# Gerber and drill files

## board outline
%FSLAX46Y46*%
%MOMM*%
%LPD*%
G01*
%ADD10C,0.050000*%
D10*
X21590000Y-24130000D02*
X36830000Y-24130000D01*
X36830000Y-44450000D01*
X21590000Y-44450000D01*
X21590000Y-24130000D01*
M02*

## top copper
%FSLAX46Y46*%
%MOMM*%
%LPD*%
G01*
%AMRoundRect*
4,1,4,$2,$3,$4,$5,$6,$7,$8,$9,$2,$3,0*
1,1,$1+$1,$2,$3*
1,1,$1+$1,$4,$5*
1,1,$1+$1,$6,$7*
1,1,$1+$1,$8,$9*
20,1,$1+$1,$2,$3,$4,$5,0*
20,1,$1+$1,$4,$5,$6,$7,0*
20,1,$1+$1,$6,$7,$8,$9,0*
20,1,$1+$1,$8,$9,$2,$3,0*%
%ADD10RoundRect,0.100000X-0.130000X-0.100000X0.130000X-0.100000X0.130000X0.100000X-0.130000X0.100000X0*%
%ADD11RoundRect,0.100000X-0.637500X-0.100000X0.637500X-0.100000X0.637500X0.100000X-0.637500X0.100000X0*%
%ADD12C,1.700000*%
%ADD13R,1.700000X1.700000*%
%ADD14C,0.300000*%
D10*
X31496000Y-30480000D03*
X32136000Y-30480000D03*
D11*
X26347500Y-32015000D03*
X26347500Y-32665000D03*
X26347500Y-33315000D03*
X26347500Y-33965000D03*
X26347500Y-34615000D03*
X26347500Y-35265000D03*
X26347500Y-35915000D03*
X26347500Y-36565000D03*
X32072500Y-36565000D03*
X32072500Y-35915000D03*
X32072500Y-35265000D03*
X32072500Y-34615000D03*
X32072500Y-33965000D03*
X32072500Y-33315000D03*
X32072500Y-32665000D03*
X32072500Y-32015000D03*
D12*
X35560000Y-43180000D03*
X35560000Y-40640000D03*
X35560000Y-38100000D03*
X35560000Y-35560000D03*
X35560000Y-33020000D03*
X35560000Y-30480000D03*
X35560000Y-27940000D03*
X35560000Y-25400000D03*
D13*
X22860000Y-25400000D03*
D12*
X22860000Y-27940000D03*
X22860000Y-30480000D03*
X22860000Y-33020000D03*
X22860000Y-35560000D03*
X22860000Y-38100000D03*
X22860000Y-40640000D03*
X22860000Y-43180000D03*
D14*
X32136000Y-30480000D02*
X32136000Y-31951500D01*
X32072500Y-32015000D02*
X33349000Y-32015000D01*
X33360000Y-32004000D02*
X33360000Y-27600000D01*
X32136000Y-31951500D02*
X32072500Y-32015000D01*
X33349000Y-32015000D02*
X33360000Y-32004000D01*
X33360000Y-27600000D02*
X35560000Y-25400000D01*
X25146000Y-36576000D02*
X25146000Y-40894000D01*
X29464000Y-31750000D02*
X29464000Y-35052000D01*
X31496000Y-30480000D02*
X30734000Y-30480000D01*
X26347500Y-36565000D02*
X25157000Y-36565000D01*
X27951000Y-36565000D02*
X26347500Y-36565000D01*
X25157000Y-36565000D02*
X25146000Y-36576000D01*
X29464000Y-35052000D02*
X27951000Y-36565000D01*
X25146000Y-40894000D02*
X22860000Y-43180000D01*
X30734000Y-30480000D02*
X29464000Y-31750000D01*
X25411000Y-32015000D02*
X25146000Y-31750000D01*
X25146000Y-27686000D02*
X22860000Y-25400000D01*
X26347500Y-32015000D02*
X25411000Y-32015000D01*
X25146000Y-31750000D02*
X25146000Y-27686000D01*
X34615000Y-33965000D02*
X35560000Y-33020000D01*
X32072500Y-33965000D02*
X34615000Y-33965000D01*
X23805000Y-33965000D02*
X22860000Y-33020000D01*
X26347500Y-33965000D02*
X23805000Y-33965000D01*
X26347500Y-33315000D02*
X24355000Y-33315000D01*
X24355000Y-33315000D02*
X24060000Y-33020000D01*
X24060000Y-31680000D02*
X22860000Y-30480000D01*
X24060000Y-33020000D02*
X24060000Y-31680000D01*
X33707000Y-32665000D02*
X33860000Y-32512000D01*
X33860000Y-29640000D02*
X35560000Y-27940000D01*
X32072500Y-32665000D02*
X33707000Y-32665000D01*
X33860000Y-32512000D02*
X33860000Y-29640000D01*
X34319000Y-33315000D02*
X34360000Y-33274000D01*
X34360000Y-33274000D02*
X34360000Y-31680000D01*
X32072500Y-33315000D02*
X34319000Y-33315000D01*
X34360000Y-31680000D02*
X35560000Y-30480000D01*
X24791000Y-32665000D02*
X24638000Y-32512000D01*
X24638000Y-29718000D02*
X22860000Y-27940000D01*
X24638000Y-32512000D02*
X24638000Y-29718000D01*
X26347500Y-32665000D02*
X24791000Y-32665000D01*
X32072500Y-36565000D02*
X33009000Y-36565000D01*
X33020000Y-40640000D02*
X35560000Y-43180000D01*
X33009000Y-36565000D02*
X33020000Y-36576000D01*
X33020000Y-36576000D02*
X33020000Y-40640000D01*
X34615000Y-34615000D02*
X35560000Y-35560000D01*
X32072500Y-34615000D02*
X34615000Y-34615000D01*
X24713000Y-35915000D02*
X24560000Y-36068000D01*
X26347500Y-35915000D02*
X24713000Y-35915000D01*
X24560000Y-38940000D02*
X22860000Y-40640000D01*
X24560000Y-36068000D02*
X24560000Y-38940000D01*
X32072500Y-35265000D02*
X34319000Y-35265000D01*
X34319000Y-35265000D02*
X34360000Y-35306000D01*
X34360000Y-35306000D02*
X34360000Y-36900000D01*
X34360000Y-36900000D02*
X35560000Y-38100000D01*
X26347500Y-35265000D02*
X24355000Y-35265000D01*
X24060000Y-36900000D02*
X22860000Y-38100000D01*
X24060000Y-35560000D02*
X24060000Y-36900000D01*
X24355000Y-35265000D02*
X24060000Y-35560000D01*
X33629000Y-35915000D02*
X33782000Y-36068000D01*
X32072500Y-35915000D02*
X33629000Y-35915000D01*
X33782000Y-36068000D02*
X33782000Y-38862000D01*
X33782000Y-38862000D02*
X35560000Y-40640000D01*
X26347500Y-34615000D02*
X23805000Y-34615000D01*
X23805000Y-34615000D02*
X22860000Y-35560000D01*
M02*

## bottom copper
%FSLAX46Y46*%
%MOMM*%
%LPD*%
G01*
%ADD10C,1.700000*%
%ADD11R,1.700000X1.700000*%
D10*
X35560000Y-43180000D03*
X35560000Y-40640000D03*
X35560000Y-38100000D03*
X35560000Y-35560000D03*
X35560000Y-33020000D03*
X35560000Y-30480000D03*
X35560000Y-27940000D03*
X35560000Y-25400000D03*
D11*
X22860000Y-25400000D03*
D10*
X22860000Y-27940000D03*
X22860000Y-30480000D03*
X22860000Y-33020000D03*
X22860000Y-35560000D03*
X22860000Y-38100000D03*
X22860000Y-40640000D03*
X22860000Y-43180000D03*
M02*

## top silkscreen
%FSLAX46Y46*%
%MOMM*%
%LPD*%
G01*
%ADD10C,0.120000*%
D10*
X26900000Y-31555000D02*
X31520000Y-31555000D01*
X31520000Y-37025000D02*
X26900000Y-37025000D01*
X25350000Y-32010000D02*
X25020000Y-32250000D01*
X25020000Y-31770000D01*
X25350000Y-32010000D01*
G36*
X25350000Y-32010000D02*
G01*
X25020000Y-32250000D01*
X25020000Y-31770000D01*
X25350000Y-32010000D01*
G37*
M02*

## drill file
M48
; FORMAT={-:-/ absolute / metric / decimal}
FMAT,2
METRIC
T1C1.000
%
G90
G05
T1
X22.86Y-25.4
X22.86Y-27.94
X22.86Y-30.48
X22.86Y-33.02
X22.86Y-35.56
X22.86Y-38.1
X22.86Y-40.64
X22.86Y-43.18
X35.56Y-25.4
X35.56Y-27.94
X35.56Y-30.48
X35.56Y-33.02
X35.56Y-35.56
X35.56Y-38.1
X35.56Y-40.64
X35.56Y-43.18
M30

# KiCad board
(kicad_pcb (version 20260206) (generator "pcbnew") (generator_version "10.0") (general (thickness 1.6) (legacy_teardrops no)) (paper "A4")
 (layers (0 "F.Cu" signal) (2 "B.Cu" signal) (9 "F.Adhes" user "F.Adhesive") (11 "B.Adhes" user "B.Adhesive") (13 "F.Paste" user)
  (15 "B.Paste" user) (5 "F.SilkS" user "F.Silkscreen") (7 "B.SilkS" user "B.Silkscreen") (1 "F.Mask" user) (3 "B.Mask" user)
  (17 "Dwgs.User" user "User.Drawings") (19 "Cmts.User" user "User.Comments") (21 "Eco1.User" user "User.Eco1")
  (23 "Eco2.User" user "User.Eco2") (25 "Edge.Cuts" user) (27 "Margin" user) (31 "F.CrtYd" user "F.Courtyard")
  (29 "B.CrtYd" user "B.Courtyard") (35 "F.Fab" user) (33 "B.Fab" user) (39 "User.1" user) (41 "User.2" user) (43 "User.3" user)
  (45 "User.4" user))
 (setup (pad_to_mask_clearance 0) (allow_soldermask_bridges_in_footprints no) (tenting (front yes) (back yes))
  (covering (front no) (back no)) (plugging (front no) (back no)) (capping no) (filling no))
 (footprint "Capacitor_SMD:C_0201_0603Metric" (layer "F.Cu") (at 31.816 30.48)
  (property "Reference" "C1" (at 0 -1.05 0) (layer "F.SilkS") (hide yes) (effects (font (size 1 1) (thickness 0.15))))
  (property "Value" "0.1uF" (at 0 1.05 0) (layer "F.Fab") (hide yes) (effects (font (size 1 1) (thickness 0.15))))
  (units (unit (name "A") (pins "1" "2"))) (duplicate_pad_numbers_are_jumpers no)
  (pad "" smd roundrect (at -0.345 0) (size 0.318 0.36) (layers "F.Paste") (roundrect_rratio 0.25))
  (pad "" smd roundrect (at 0.345 0) (size 0.318 0.36) (layers "F.Paste") (roundrect_rratio 0.25))
  (pad "1" smd roundrect (at -0.32 0) (size 0.46 0.4) (layers "F.Cu" "F.Mask") (roundrect_rratio 0.25) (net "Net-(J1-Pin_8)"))
  (pad "2" smd roundrect (at 0.32 0) (size 0.46 0.4) (layers "F.Cu" "F.Mask") (roundrect_rratio 0.25) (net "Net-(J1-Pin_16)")))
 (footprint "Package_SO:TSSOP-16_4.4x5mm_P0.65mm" (layer "F.Cu") (at 29.21 34.29)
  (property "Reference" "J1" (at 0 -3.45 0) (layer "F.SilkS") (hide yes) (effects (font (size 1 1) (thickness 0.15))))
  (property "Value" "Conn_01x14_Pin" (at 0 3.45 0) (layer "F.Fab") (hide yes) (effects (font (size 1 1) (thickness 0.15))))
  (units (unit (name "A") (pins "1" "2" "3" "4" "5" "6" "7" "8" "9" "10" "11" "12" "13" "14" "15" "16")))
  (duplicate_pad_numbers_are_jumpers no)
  (fp_line (start -2.31 -2.735) (end 2.31 -2.735) (stroke (width 0.12) (type solid)) (layer "F.SilkS"))
  (fp_line (start 2.31 2.735) (end -2.31 2.735) (stroke (width 0.12) (type solid)) (layer "F.SilkS"))
  (fp_poly (pts (xy -3.86 -2.28) (xy -4.19 -2.04) (xy -4.19 -2.52)) (stroke (width 0.12) (type solid)) (fill yes) (layer "F.SilkS"))
  (pad "1" smd roundrect (at -2.8625 -2.275) (size 1.475 0.4) (layers "F.Cu" "F.Mask" "F.Paste") (roundrect_rratio 0.25)
   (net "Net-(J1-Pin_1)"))
  (pad "2" smd roundrect (at -2.8625 -1.625) (size 1.475 0.4) (layers "F.Cu" "F.Mask" "F.Paste") (roundrect_rratio 0.25)
   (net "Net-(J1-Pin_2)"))
  (pad "3" smd roundrect (at -2.8625 -0.975) (size 1.475 0.4) (layers "F.Cu" "F.Mask" "F.Paste") (roundrect_rratio 0.25)
   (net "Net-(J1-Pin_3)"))
  (pad "4" smd roundrect (at -2.8625 -0.325) (size 1.475 0.4) (layers "F.Cu" "F.Mask" "F.Paste") (roundrect_rratio 0.25)
   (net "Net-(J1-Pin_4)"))
  (pad "5" smd roundrect (at -2.8625 0.325) (size 1.475 0.4) (layers "F.Cu" "F.Mask" "F.Paste") (roundrect_rratio 0.25)
   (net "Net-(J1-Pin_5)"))
  (pad "6" smd roundrect (at -2.8625 0.975) (size 1.475 0.4) (layers "F.Cu" "F.Mask" "F.Paste") (roundrect_rratio 0.25)
   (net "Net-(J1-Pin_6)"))
  (pad "7" smd roundrect (at -2.8625 1.625) (size 1.475 0.4) (layers "F.Cu" "F.Mask" "F.Paste") (roundrect_rratio 0.25)
   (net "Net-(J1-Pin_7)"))
  (pad "8" smd roundrect (at -2.8625 2.275) (size 1.475 0.4) (layers "F.Cu" "F.Mask" "F.Paste") (roundrect_rratio 0.25)
   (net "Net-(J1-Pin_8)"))
  (pad "9" smd roundrect (at 2.8625 2.275) (size 1.475 0.4) (layers "F.Cu" "F.Mask" "F.Paste") (roundrect_rratio 0.25)
   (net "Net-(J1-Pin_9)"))
  (pad "10" smd roundrect (at 2.8625 1.625) (size 1.475 0.4) (layers "F.Cu" "F.Mask" "F.Paste") (roundrect_rratio 0.25)
   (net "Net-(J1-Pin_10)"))
  (pad "11" smd roundrect (at 2.8625 0.975) (size 1.475 0.4) (layers "F.Cu" "F.Mask" "F.Paste") (roundrect_rratio 0.25)
   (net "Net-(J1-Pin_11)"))
  (pad "12" smd roundrect (at 2.8625 0.325) (size 1.475 0.4) (layers "F.Cu" "F.Mask" "F.Paste") (roundrect_rratio 0.25)
   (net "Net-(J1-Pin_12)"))
  (pad "13" smd roundrect (at 2.8625 -0.325) (size 1.475 0.4) (layers "F.Cu" "F.Mask" "F.Paste") (roundrect_rratio 0.25)
   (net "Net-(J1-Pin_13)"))
  (pad "14" smd roundrect (at 2.8625 -0.975) (size 1.475 0.4) (layers "F.Cu" "F.Mask" "F.Paste") (roundrect_rratio 0.25)
   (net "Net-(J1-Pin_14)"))
  (pad "15" smd roundrect (at 2.8625 -1.625) (size 1.475 0.4) (layers "F.Cu" "F.Mask" "F.Paste") (roundrect_rratio 0.25)
   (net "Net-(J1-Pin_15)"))
  (pad "16" smd roundrect (at 2.8625 -2.275) (size 1.475 0.4) (layers "F.Cu" "F.Mask" "F.Paste") (roundrect_rratio 0.25)
   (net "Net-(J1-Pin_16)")))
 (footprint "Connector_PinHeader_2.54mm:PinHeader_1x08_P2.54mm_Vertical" (layer "B.Cu") (at 35.56 43.18)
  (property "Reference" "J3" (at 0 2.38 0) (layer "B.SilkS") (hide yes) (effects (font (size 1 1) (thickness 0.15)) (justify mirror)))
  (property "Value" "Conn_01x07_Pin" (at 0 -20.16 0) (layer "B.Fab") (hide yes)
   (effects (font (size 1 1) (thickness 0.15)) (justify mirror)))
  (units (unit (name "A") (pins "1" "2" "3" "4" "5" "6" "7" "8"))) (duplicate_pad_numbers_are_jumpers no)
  (pad "1" thru_hole circle (at 0 0) (size 1.7 1.7) (drill 1) (layers "*.Cu" "*.Mask") (remove_unused_layers no) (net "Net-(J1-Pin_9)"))
  (pad "2" thru_hole circle (at 0 -2.54) (size 1.7 1.7) (drill 1) (layers "*.Cu" "*.Mask") (remove_unused_layers no) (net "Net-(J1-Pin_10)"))
  (pad "3" thru_hole circle (at 0 -5.08) (size 1.7 1.7) (drill 1) (layers "*.Cu" "*.Mask") (remove_unused_layers no) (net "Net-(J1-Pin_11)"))
  (pad "4" thru_hole circle (at 0 -7.62) (size 1.7 1.7) (drill 1) (layers "*.Cu" "*.Mask") (remove_unused_layers no) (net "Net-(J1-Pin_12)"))
  (pad "5" thru_hole circle (at 0 -10.16) (size 1.7 1.7) (drill 1) (layers "*.Cu" "*.Mask") (remove_unused_layers no)
   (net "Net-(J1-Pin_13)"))
  (pad "6" thru_hole circle (at 0 -12.7) (size 1.7 1.7) (drill 1) (layers "*.Cu" "*.Mask") (remove_unused_layers no) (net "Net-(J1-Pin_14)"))
  (pad "7" thru_hole circle (at 0 -15.24) (size 1.7 1.7) (drill 1) (layers "*.Cu" "*.Mask") (remove_unused_layers no)
   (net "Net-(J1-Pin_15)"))
  (pad "8" thru_hole circle (at 0 -17.78) (size 1.7 1.7) (drill 1) (layers "*.Cu" "*.Mask") (remove_unused_layers no)
   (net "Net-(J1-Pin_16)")))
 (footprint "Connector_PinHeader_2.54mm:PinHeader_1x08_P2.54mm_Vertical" (layer "B.Cu") (at 22.86 25.4 180)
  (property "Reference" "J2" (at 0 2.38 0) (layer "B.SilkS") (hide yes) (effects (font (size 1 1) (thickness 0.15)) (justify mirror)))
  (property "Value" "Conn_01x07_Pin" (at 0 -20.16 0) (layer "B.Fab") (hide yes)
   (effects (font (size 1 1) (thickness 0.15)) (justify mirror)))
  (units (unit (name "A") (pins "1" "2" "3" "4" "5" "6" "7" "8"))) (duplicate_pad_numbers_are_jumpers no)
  (pad "1" thru_hole rect (at 0 0 180) (size 1.7 1.7) (drill 1) (layers "*.Cu" "*.Mask") (remove_unused_layers no) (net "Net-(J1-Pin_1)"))
  (pad "2" thru_hole circle (at 0 -2.54 180) (size 1.7 1.7) (drill 1) (layers "*.Cu" "*.Mask") (remove_unused_layers no)
   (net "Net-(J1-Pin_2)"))
  (pad "3" thru_hole circle (at 0 -5.08 180) (size 1.7 1.7) (drill 1) (layers "*.Cu" "*.Mask") (remove_unused_layers no)
   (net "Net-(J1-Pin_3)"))
  (pad "4" thru_hole circle (at 0 -7.62 180) (size 1.7 1.7) (drill 1) (layers "*.Cu" "*.Mask") (remove_unused_layers no)
   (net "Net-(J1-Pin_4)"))
  (pad "5" thru_hole circle (at 0 -10.16 180) (size 1.7 1.7) (drill 1) (layers "*.Cu" "*.Mask") (remove_unused_layers no)
   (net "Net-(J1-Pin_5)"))
  (pad "6" thru_hole circle (at 0 -12.7 180) (size 1.7 1.7) (drill 1) (layers "*.Cu" "*.Mask") (remove_unused_layers no)
   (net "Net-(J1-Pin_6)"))
  (pad "7" thru_hole circle (at 0 -15.24 180) (size 1.7 1.7) (drill 1) (layers "*.Cu" "*.Mask") (remove_unused_layers no)
   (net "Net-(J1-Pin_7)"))
  (pad "8" thru_hole circle (at 0 -17.78 180) (size 1.7 1.7) (drill 1) (layers "*.Cu" "*.Mask") (remove_unused_layers no)
   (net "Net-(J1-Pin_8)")))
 (gr_rect (start 21.59 24.13) (end 36.83 44.45) (stroke (width 0.05) (type default)) (fill no) (layer "Edge.Cuts"))
 (segment (start 32.136 30.48) (end 32.136 31.9515) (width 0.3) (layer "F.Cu") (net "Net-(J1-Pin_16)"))
 (segment (start 32.0725 32.015) (end 33.349 32.015) (width 0.3) (layer "F.Cu") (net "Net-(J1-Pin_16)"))
 (segment (start 33.36 32.004) (end 33.36 27.6) (width 0.3) (layer "F.Cu") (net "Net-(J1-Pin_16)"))
 (segment (start 32.136 31.9515) (end 32.0725 32.015) (width 0.3) (layer "F.Cu") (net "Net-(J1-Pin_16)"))
 (segment (start 33.349 32.015) (end 33.36 32.004) (width 0.3) (layer "F.Cu") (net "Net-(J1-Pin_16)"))
 (segment (start 33.36 27.6) (end 35.56 25.4) (width 0.3) (layer "F.Cu") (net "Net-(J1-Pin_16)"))
 (segment (start 25.146 36.576) (end 25.146 40.894) (width 0.3) (layer "F.Cu") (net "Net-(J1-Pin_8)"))
 (segment (start 29.464 31.75) (end 29.464 35.052) (width 0.3) (layer "F.Cu") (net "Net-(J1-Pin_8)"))
 (segment (start 31.496 30.48) (end 30.734 30.48) (width 0.3) (layer "F.Cu") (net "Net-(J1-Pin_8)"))
 (segment (start 26.3475 36.565) (end 25.157 36.565) (width 0.3) (layer "F.Cu") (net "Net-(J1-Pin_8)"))
 (segment (start 27.951 36.565) (end 26.3475 36.565) (width 0.3) (layer "F.Cu") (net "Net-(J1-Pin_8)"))
 (segment (start 25.157 36.565) (end 25.146 36.576) (width 0.3) (layer "F.Cu") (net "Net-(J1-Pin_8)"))
 (segment (start 29.464 35.052) (end 27.951 36.565) (width 0.3) (layer "F.Cu") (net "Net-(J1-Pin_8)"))
 (segment (start 25.146 40.894) (end 22.86 43.18) (width 0.3) (layer "F.Cu") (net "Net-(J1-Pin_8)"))
 (segment (start 30.734 30.48) (end 29.464 31.75) (width 0.3) (layer "F.Cu") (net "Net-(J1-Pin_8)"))
 (segment (start 25.411 32.015) (end 25.146 31.75) (width 0.3) (layer "F.Cu") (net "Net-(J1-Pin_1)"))
 (segment (start 25.146 27.686) (end 22.86 25.4) (width 0.3) (layer "F.Cu") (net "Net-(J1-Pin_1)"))
 (segment (start 26.3475 32.015) (end 25.411 32.015) (width 0.3) (layer "F.Cu") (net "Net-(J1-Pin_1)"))
 (segment (start 25.146 31.75) (end 25.146 27.686) (width 0.3) (layer "F.Cu") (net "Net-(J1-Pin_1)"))
 (segment (start 34.615 33.965) (end 35.56 33.02) (width 0.3) (layer "F.Cu") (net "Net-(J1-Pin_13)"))
 (segment (start 32.0725 33.965) (end 34.615 33.965) (width 0.3) (layer "F.Cu") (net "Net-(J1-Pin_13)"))
 (segment (start 23.805 33.965) (end 22.86 33.02) (width 0.3) (layer "F.Cu") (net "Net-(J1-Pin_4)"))
 (segment (start 26.3475 33.965) (end 23.805 33.965) (width 0.3) (layer "F.Cu") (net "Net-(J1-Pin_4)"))
 (segment (start 26.3475 33.315) (end 24.355 33.315) (width 0.3) (layer "F.Cu") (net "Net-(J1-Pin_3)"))
 (segment (start 24.355 33.315) (end 24.06 33.02) (width 0.3) (layer "F.Cu") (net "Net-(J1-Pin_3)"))
 (segment (start 24.06 31.68) (end 22.86 30.48) (width 0.3) (layer "F.Cu") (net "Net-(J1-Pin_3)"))
 (segment (start 24.06 33.02) (end 24.06 31.68) (width 0.3) (layer "F.Cu") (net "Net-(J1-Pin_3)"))
 (segment (start 33.707 32.665) (end 33.86 32.512) (width 0.3) (layer "F.Cu") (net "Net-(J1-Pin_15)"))
 (segment (start 33.86 29.64) (end 35.56 27.94) (width 0.3) (layer "F.Cu") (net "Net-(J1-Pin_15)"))
 (segment (start 32.0725 32.665) (end 33.707 32.665) (width 0.3) (layer "F.Cu") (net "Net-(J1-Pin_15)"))
 (segment (start 33.86 32.512) (end 33.86 29.64) (width 0.3) (layer "F.Cu") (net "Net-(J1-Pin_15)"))
 (segment (start 34.319 33.315) (end 34.36 33.274) (width 0.3) (layer "F.Cu") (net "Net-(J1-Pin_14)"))
 (segment (start 34.36 33.274) (end 34.36 31.68) (width 0.3) (layer "F.Cu") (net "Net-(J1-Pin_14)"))
 (segment (start 32.0725 33.315) (end 34.319 33.315) (width 0.3) (layer "F.Cu") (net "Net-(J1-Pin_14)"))
 (segment (start 34.36 31.68) (end 35.56 30.48) (width 0.3) (layer "F.Cu") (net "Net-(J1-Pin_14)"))
 (segment (start 24.791 32.665) (end 24.638 32.512) (width 0.3) (layer "F.Cu") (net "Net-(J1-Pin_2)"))
 (segment (start 24.638 29.718) (end 22.86 27.94) (width 0.3) (layer "F.Cu") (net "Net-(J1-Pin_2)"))
 (segment (start 24.638 32.512) (end 24.638 29.718) (width 0.3) (layer "F.Cu") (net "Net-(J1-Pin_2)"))
 (segment (start 26.3475 32.665) (end 24.791 32.665) (width 0.3) (layer "F.Cu") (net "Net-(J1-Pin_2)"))
 (segment (start 32.0725 36.565) (end 33.009 36.565) (width 0.3) (layer "F.Cu") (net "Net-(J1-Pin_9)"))
 (segment (start 33.02 40.64) (end 35.56 43.18) (width 0.3) (layer "F.Cu") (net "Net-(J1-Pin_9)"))
 (segment (start 33.009 36.565) (end 33.02 36.576) (width 0.3) (layer "F.Cu") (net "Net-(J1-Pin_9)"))
 (segment (start 33.02 36.576) (end 33.02 40.64) (width 0.3) (layer "F.Cu") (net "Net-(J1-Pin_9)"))
 (segment (start 34.615 34.615) (end 35.56 35.56) (width 0.3) (layer "F.Cu") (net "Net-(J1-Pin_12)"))
 (segment (start 32.0725 34.615) (end 34.615 34.615) (width 0.3) (layer "F.Cu") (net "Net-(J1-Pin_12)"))
 (segment (start 24.713 35.915) (end 24.56 36.068) (width 0.3) (layer "F.Cu") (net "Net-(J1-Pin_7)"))
 (segment (start 26.3475 35.915) (end 24.713 35.915) (width 0.3) (layer "F.Cu") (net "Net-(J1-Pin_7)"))
 (segment (start 24.56 38.94) (end 22.86 40.64) (width 0.3) (layer "F.Cu") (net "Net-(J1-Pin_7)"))
 (segment (start 24.56 36.068) (end 24.56 38.94) (width 0.3) (layer "F.Cu") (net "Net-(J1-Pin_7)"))
 (segment (start 32.0725 35.265) (end 34.319 35.265) (width 0.3) (layer "F.Cu") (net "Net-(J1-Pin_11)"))
 (segment (start 34.319 35.265) (end 34.36 35.306) (width 0.3) (layer "F.Cu") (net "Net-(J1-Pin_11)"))
 (segment (start 34.36 35.306) (end 34.36 36.9) (width 0.3) (layer "F.Cu") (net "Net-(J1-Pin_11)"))
 (segment (start 34.36 36.9) (end 35.56 38.1) (width 0.3) (layer "F.Cu") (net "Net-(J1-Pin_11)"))
 (segment (start 26.3475 35.265) (end 24.355 35.265) (width 0.3) (layer "F.Cu") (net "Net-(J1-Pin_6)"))
 (segment (start 24.06 36.9) (end 22.86 38.1) (width 0.3) (layer "F.Cu") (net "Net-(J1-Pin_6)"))
 (segment (start 24.06 35.56) (end 24.06 36.9) (width 0.3) (layer "F.Cu") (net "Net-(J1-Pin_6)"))
 (segment (start 24.355 35.265) (end 24.06 35.56) (width 0.3) (layer "F.Cu") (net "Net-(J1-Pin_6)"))
 (segment (start 33.629 35.915) (end 33.782 36.068) (width 0.3) (layer "F.Cu") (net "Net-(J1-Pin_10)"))
 (segment (start 32.0725 35.915) (end 33.629 35.915) (width 0.3) (layer "F.Cu") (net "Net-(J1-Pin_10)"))
 (segment (start 33.782 36.068) (end 33.782 38.862) (width 0.3) (layer "F.Cu") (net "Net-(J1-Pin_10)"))
 (segment (start 33.782 38.862) (end 35.56 40.64) (width 0.3) (layer "F.Cu") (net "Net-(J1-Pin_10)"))
 (segment (start 26.3475 34.615) (end 23.805 34.615) (width 0.3) (layer "F.Cu") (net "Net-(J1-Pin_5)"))
 (segment (start 23.805 34.615) (end 22.86 35.56) (width 0.3) (layer "F.Cu") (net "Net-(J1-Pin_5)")))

